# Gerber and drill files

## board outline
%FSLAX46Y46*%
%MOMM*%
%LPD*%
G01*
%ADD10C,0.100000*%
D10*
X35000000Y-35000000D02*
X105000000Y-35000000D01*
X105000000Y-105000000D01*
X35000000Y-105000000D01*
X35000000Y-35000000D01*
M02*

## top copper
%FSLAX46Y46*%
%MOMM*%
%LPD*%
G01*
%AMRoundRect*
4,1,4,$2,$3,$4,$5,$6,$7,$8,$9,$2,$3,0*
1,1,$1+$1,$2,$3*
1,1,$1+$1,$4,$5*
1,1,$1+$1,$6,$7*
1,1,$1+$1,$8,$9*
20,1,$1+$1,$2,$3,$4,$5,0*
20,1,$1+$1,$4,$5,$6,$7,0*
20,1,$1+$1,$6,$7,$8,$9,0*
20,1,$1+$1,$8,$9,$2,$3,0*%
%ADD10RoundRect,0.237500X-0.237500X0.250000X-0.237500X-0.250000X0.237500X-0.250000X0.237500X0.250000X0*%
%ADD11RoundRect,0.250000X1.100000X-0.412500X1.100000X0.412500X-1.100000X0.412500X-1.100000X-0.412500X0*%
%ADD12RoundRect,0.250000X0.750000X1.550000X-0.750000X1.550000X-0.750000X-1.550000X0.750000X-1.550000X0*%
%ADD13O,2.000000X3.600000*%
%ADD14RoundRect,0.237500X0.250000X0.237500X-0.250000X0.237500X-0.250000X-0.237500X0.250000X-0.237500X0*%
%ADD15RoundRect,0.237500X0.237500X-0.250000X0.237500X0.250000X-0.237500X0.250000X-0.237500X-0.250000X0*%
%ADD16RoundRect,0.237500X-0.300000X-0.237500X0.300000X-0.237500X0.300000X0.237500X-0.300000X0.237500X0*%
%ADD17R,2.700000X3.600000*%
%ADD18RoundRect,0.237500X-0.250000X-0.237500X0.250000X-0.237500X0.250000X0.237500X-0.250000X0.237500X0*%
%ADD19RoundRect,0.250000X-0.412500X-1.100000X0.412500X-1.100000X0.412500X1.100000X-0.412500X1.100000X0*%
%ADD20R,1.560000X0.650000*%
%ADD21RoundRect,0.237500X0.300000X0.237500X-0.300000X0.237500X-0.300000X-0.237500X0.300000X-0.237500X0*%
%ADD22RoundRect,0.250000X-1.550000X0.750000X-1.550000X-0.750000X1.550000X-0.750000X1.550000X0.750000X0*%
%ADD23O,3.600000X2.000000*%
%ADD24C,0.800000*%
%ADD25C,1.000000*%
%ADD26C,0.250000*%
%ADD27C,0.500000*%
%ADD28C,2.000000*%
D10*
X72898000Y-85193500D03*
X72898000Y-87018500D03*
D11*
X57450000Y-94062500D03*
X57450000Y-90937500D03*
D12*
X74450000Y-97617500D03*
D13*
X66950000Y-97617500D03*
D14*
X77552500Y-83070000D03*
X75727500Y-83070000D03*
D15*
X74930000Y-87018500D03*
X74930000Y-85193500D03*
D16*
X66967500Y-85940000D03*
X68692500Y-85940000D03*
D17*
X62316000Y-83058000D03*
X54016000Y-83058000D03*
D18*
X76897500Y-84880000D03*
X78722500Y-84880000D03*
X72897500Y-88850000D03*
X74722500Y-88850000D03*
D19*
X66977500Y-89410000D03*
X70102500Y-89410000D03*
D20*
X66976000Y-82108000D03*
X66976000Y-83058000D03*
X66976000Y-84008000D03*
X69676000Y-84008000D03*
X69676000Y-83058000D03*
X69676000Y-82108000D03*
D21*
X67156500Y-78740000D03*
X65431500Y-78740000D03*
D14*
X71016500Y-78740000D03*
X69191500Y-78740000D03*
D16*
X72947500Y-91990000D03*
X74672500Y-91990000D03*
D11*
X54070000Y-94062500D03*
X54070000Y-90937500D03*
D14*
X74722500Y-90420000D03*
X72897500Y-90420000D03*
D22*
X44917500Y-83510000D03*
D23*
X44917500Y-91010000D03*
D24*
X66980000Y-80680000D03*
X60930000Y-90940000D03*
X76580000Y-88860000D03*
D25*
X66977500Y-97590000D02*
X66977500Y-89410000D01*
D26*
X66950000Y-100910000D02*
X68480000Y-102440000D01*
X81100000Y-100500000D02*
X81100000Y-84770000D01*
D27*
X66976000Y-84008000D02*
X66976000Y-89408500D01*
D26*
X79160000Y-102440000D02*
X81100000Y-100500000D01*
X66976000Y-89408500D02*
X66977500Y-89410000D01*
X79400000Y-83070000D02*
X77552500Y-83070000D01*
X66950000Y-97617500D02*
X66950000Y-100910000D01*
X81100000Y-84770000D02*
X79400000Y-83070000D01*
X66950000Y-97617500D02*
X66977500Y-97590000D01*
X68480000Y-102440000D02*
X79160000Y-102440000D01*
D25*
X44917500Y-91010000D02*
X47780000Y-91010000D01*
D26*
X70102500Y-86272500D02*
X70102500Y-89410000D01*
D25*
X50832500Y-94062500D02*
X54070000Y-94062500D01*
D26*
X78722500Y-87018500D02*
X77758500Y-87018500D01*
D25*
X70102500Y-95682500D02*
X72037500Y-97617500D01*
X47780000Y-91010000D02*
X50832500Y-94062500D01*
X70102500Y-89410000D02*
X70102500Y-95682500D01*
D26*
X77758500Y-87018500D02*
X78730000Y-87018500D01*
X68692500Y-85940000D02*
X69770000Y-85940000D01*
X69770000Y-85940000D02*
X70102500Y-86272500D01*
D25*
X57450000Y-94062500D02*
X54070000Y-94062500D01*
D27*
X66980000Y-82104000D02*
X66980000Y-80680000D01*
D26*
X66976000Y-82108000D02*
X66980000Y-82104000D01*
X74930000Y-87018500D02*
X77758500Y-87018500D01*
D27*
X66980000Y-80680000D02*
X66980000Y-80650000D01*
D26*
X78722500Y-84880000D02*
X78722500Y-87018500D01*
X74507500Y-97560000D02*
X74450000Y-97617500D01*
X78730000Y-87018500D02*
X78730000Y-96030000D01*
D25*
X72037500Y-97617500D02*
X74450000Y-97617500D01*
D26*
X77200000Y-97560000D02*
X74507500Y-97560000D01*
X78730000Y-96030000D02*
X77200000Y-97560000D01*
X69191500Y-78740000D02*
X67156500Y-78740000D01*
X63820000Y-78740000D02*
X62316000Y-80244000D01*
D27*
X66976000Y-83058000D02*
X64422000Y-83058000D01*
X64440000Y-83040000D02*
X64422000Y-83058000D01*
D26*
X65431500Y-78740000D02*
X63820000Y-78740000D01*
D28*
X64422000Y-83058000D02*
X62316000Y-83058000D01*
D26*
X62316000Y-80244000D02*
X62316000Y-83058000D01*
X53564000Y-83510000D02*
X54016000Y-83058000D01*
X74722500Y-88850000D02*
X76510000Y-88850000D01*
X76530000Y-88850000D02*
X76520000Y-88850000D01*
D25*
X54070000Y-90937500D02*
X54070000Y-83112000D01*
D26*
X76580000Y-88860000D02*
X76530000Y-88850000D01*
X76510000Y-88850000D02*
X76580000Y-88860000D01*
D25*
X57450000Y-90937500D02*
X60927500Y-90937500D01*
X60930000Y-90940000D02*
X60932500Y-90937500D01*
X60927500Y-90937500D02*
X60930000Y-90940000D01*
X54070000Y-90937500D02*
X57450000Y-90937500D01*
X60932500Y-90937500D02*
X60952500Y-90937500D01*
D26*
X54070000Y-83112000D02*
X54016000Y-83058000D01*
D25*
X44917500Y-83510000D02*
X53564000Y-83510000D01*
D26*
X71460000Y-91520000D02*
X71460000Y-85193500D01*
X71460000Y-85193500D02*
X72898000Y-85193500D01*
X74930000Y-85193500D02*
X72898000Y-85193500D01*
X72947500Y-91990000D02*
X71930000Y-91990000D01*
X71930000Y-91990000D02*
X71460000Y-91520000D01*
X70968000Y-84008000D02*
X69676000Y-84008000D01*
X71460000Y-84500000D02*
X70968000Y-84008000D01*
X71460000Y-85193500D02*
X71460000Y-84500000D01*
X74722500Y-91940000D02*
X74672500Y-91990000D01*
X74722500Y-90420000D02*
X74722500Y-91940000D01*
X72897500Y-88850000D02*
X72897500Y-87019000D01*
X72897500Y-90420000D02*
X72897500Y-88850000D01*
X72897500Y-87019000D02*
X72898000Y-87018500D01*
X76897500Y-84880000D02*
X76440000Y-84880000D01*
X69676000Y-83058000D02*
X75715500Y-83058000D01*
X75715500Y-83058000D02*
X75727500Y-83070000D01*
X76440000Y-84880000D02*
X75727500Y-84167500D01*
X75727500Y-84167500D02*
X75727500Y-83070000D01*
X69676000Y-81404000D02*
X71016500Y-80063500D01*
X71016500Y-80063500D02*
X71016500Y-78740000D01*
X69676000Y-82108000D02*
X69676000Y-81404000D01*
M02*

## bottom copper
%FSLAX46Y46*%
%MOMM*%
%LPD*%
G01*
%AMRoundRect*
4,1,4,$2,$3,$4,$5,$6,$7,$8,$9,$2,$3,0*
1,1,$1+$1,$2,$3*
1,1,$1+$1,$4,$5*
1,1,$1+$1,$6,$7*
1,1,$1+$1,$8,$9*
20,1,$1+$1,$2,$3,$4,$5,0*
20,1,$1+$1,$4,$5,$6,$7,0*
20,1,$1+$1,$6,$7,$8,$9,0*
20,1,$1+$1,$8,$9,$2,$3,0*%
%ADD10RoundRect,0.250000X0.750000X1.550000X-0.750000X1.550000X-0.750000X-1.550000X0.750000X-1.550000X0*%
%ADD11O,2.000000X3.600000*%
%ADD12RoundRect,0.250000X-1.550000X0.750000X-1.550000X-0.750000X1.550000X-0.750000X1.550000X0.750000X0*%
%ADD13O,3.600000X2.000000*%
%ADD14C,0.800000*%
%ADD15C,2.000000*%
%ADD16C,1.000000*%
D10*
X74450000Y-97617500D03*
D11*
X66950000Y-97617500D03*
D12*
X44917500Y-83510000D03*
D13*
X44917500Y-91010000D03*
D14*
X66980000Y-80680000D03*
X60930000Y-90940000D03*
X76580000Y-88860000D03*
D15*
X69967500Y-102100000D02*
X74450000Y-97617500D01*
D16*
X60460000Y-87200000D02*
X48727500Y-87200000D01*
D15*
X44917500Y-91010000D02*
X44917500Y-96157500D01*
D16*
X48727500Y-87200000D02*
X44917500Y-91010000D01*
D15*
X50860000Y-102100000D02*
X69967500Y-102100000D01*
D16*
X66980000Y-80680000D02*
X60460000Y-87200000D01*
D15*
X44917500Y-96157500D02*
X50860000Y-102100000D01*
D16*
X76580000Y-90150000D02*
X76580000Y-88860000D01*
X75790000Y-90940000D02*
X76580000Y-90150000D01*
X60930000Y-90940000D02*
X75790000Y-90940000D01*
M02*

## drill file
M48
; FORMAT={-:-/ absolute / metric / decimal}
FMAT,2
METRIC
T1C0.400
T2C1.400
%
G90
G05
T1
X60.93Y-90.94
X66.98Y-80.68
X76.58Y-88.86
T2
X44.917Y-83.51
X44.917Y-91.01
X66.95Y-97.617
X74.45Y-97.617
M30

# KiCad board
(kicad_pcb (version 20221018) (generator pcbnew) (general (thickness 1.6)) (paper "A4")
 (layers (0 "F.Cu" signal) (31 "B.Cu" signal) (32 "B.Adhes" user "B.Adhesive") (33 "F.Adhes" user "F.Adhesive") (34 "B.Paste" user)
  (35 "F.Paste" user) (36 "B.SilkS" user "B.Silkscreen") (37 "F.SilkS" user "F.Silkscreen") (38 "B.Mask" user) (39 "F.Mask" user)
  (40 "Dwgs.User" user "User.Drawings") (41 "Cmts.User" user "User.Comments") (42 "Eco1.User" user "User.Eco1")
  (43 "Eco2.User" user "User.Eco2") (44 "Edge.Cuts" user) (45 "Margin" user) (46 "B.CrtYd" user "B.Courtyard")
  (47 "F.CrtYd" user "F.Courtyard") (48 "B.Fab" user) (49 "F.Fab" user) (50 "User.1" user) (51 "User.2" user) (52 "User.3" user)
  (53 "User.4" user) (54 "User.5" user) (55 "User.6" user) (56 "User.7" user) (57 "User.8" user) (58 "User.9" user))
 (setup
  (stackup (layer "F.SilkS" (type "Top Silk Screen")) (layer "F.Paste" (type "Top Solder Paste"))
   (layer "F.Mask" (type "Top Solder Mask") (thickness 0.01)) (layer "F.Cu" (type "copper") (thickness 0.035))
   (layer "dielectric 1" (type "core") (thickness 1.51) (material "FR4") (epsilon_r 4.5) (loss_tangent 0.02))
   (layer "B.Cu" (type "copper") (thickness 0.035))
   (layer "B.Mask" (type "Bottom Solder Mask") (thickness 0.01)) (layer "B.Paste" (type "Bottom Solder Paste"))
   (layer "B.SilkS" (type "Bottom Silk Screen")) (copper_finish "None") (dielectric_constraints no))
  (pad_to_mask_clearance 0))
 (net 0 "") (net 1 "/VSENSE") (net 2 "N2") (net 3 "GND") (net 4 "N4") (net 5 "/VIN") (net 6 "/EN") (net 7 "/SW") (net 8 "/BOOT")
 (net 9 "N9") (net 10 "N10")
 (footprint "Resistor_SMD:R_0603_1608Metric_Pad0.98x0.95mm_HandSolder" (layer "F.Cu") (at 72.898 86.106 -90)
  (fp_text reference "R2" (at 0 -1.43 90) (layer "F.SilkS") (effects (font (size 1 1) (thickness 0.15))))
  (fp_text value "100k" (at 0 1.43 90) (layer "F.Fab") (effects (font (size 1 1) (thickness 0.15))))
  (pad "1" smd roundrect (at -0.9125 0 270) (size 0.975 0.95) (layers "F.Cu" "F.Paste" "F.Mask") (roundrect_rratio 0.25) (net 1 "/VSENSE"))
  (pad "2" smd roundrect (at 0.9125 0 270) (size 0.975 0.95) (layers "F.Cu" "F.Paste" "F.Mask") (roundrect_rratio 0.25) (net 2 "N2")))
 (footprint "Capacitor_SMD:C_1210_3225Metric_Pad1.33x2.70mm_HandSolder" (layer "F.Cu") (at 57.45 92.5 90)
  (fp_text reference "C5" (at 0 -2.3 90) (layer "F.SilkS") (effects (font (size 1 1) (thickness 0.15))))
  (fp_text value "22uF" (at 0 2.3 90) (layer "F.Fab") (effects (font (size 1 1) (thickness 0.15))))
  (pad "1" smd roundrect (at -1.5625 0 90) (size 1.325 2.7) (layers "F.Cu" "F.Paste" "F.Mask") (roundrect_rratio 0.188679) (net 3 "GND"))
  (pad "2" smd roundrect (at 1.5625 0 90) (size 1.325 2.7) (layers "F.Cu" "F.Paste" "F.Mask") (roundrect_rratio 0.188679) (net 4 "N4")))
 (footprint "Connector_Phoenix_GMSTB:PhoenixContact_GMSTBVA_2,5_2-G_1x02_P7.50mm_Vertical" (layer "F.Cu") (at 70.76 97.6175 180)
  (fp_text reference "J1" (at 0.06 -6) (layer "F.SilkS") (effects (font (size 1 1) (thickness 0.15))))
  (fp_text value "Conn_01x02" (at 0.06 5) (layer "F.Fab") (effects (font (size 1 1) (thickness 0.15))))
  (pad "1" thru_hole roundrect (at -3.69 0 180) (size 2 3.6) (drill 1.4) (layers "*.Cu" "*.Mask") (roundrect_rratio 0.125) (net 3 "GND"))
  (pad "2" thru_hole oval (at 3.81 0 180) (size 2 3.6) (drill 1.4) (layers "*.Cu" "*.Mask") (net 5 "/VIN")))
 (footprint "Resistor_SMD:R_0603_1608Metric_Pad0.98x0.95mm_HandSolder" (layer "F.Cu") (at 76.64 83.07 180)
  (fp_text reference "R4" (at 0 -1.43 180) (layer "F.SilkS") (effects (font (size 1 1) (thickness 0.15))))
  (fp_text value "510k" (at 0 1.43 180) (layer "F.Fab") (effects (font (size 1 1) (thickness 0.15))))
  (pad "1" smd roundrect (at -0.9125 0 180) (size 0.975 0.95) (layers "F.Cu" "F.Paste" "F.Mask") (roundrect_rratio 0.25) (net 5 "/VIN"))
  (pad "2" smd roundrect (at 0.9125 0 180) (size 0.975 0.95) (layers "F.Cu" "F.Paste" "F.Mask") (roundrect_rratio 0.25) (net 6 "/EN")))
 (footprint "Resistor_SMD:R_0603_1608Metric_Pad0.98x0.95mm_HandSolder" (layer "F.Cu") (at 74.93 86.106 90)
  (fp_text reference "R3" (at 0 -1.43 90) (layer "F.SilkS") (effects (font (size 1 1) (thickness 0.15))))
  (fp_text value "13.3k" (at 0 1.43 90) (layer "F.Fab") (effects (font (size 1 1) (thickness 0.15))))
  (pad "1" smd roundrect (at -0.9125 0 90) (size 0.975 0.95) (layers "F.Cu" "F.Paste" "F.Mask") (roundrect_rratio 0.25) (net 3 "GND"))
  (pad "2" smd roundrect (at 0.9125 0 90) (size 0.975 0.95) (layers "F.Cu" "F.Paste" "F.Mask") (roundrect_rratio 0.25) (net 1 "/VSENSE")))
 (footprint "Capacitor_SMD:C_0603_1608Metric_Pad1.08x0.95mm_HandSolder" (layer "F.Cu") (at 67.83 85.94)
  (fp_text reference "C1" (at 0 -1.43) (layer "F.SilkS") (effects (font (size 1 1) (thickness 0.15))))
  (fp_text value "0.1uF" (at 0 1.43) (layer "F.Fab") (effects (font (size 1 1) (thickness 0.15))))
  (pad "1" smd roundrect (at -0.8625 0) (size 1.075 0.95) (layers "F.Cu" "F.Paste" "F.Mask") (roundrect_rratio 0.25) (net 5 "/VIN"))
  (pad "2" smd roundrect (at 0.8625 0) (size 1.075 0.95) (layers "F.Cu" "F.Paste" "F.Mask") (roundrect_rratio 0.25) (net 3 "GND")))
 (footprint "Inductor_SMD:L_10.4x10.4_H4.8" (layer "F.Cu") (at 58.166 83.058 180)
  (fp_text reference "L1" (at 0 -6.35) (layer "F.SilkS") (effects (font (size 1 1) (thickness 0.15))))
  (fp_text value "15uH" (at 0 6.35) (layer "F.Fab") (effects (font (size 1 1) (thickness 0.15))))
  (pad "1" smd rect (at -4.15 0 180) (size 2.7 3.6) (layers "F.Cu" "F.Paste" "F.Mask") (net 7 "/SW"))
  (pad "2" smd rect (at 4.15 0 180) (size 2.7 3.6) (layers "F.Cu" "F.Paste" "F.Mask") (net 4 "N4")))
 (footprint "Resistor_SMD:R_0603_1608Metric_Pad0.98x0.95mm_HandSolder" (layer "F.Cu") (at 77.81 84.88)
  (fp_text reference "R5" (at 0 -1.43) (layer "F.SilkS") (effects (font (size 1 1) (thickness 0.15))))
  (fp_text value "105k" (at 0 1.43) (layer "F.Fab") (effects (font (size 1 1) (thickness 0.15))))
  (pad "1" smd roundrect (at -0.9125 0) (size 0.975 0.95) (layers "F.Cu" "F.Paste" "F.Mask") (roundrect_rratio 0.25) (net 6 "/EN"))
  (pad "2" smd roundrect (at 0.9125 0) (size 0.975 0.95) (layers "F.Cu" "F.Paste" "F.Mask") (roundrect_rratio 0.25) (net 3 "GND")))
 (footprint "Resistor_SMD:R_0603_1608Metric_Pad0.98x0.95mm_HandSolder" (layer "F.Cu") (at 73.81 88.85)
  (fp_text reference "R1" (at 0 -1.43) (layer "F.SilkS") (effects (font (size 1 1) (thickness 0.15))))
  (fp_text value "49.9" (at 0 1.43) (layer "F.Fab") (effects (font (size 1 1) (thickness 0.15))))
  (pad "1" smd roundrect (at -0.9125 0) (size 0.975 0.95) (layers "F.Cu" "F.Paste" "F.Mask") (roundrect_rratio 0.25) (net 2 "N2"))
  (pad "2" smd roundrect (at 0.9125 0) (size 0.975 0.95) (layers "F.Cu" "F.Paste" "F.Mask") (roundrect_rratio 0.25) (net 4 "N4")))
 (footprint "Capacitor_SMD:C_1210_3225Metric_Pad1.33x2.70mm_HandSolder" (layer "F.Cu") (at 68.54 89.41)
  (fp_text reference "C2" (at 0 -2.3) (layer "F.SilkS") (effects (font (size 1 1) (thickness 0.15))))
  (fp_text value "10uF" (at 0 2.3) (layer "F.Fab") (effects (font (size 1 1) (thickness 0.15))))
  (pad "1" smd roundrect (at -1.5625 0) (size 1.325 2.7) (layers "F.Cu" "F.Paste" "F.Mask") (roundrect_rratio 0.188679) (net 5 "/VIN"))
  (pad "2" smd roundrect (at 1.5625 0) (size 1.325 2.7) (layers "F.Cu" "F.Paste" "F.Mask") (roundrect_rratio 0.188679) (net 3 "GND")))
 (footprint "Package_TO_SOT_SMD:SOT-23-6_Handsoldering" (layer "F.Cu") (at 68.326 83.058)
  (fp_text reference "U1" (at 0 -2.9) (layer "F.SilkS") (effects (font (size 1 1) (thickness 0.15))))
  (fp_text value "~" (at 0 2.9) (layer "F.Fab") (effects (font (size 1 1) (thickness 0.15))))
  (pad "1" smd rect (at -1.35 -0.95) (size 1.56 0.65) (layers "F.Cu" "F.Paste" "F.Mask") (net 3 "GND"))
  (pad "2" smd rect (at -1.35 0) (size 1.56 0.65) (layers "F.Cu" "F.Paste" "F.Mask") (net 7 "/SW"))
  (pad "3" smd rect (at -1.35 0.95) (size 1.56 0.65) (layers "F.Cu" "F.Paste" "F.Mask") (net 5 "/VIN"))
  (pad "4" smd rect (at 1.35 0.95) (size 1.56 0.65) (layers "F.Cu" "F.Paste" "F.Mask") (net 1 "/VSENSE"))
  (pad "5" smd rect (at 1.35 0) (size 1.56 0.65) (layers "F.Cu" "F.Paste" "F.Mask") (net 6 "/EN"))
  (pad "6" smd rect (at 1.35 -0.95) (size 1.56 0.65) (layers "F.Cu" "F.Paste" "F.Mask") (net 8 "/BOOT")))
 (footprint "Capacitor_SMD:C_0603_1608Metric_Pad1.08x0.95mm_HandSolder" (layer "F.Cu") (at 66.294 78.74 180)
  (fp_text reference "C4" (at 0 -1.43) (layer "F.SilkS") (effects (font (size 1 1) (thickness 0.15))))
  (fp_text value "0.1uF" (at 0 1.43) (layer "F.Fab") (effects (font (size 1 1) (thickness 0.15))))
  (pad "1" smd roundrect (at -0.8625 0 180) (size 1.075 0.95) (layers "F.Cu" "F.Paste" "F.Mask") (roundrect_rratio 0.25) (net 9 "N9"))
  (pad "2" smd roundrect (at 0.8625 0 180) (size 1.075 0.95) (layers "F.Cu" "F.Paste" "F.Mask") (roundrect_rratio 0.25) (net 7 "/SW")))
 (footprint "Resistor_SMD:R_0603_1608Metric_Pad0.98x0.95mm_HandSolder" (layer "F.Cu") (at 70.104 78.74 180)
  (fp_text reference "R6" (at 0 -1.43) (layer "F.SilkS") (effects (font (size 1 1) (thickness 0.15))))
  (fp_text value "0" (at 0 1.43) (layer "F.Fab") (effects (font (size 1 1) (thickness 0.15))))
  (pad "1" smd roundrect (at -0.9125 0 180) (size 0.975 0.95) (layers "F.Cu" "F.Paste" "F.Mask") (roundrect_rratio 0.25) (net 8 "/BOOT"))
  (pad "2" smd roundrect (at 0.9125 0 180) (size 0.975 0.95) (layers "F.Cu" "F.Paste" "F.Mask") (roundrect_rratio 0.25) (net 9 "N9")))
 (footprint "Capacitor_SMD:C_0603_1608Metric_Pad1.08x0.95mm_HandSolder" (layer "F.Cu") (at 73.81 91.99)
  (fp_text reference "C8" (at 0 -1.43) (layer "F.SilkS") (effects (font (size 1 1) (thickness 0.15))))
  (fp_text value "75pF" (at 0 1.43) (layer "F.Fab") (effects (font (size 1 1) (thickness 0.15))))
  (pad "1" smd roundrect (at -0.8625 0) (size 1.075 0.95) (layers "F.Cu" "F.Paste" "F.Mask") (roundrect_rratio 0.25) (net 1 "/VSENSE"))
  (pad "2" smd roundrect (at 0.8625 0) (size 1.075 0.95) (layers "F.Cu" "F.Paste" "F.Mask") (roundrect_rratio 0.25) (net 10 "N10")))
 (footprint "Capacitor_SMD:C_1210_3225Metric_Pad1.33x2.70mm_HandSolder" (layer "F.Cu") (at 54.07 92.5 90)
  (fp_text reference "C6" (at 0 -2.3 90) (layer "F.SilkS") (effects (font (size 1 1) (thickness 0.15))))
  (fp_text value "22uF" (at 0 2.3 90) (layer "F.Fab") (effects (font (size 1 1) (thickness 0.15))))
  (pad "1" smd roundrect (at -1.5625 0 90) (size 1.325 2.7) (layers "F.Cu" "F.Paste" "F.Mask") (roundrect_rratio 0.188679) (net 3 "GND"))
  (pad "2" smd roundrect (at 1.5625 0 90) (size 1.325 2.7) (layers "F.Cu" "F.Paste" "F.Mask") (roundrect_rratio 0.188679) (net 4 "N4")))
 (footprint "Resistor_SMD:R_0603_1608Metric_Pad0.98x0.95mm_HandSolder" (layer "F.Cu") (at 73.81 90.42 180)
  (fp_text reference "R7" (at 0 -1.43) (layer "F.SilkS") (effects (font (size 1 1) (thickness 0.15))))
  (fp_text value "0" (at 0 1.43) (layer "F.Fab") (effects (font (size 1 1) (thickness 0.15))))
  (pad "1" smd roundrect (at -0.9125 0 180) (size 0.975 0.95) (layers "F.Cu" "F.Paste" "F.Mask") (roundrect_rratio 0.25) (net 10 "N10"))
  (pad "2" smd roundrect (at 0.9125 0 180) (size 0.975 0.95) (layers "F.Cu" "F.Paste" "F.Mask") (roundrect_rratio 0.25) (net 2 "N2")))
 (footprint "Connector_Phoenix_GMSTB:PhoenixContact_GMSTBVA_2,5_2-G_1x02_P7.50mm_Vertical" (layer "F.Cu") (at 44.9175 87.2 -90)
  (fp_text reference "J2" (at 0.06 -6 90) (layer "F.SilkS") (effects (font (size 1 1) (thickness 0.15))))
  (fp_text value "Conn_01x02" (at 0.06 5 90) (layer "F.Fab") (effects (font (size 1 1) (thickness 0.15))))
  (pad "1" thru_hole roundrect (at -3.69 0 270) (size 2 3.6) (drill 1.4) (layers "*.Cu" "*.Mask") (roundrect_rratio 0.125) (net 4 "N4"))
  (pad "2" thru_hole oval (at 3.81 0 270) (size 2 3.6) (drill 1.4) (layers "*.Cu" "*.Mask") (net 3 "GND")))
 (gr_rect (start 35 35) (end 105 105) (stroke (width 0.1) (type default)) (fill none) (layer "Edge.Cuts"))
 (segment (start 66.9775 97.59) (end 66.9775 89.41) (width 1) (layer "F.Cu") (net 5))
 (segment (start 66.95 100.91) (end 68.48 102.44) (width 0.25) (layer "F.Cu") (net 5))
 (segment (start 81.1 100.5) (end 81.1 84.77) (width 0.25) (layer "F.Cu") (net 5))
 (segment (start 66.976 84.008) (end 66.976 89.4085) (width 0.5) (layer "F.Cu") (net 5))
 (segment (start 79.16 102.44) (end 81.1 100.5) (width 0.25) (layer "F.Cu") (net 5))
 (segment (start 66.976 89.4085) (end 66.9775 89.41) (width 0.25) (layer "F.Cu") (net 5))
 (segment (start 79.4 83.07) (end 77.5525 83.07) (width 0.25) (layer "F.Cu") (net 5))
 (segment (start 66.95 97.6175) (end 66.95 100.91) (width 0.25) (layer "F.Cu") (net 5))
 (segment (start 81.1 84.77) (end 79.4 83.07) (width 0.25) (layer "F.Cu") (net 5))
 (segment (start 66.95 97.6175) (end 66.9775 97.59) (width 0.25) (layer "F.Cu") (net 5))
 (segment (start 68.48 102.44) (end 79.16 102.44) (width 0.25) (layer "F.Cu") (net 5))
 (segment (start 44.9175 91.01) (end 47.78 91.01) (width 1) (layer "F.Cu") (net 3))
 (segment (start 70.1025 86.2725) (end 70.1025 89.41) (width 0.25) (layer "F.Cu") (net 3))
 (segment (start 50.8325 94.0625) (end 54.07 94.0625) (width 1) (layer "F.Cu") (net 3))
 (segment (start 78.7225 87.0185) (end 77.7585 87.0185) (width 0.25) (layer "F.Cu") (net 3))
 (segment (start 70.1025 95.6825) (end 72.0375 97.6175) (width 1) (layer "F.Cu") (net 3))
 (segment (start 47.78 91.01) (end 50.8325 94.0625) (width 1) (layer "F.Cu") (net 3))
 (segment (start 70.1025 89.41) (end 70.1025 95.6825) (width 1) (layer "F.Cu") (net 3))
 (segment (start 77.7585 87.0185) (end 78.73 87.0185) (width 0.25) (layer "F.Cu") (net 3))
 (segment (start 68.6925 85.94) (end 69.77 85.94) (width 0.25) (layer "F.Cu") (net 3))
 (segment (start 69.77 85.94) (end 70.1025 86.2725) (width 0.25) (layer "F.Cu") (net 3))
 (segment (start 57.45 94.0625) (end 54.07 94.0625) (width 1) (layer "F.Cu") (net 3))
 (segment (start 66.98 82.104) (end 66.98 80.68) (width 0.5) (layer "F.Cu") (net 3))
 (segment (start 66.976 82.108) (end 66.98 82.104) (width 0.25) (layer "F.Cu") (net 3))
 (segment (start 74.93 87.0185) (end 77.7585 87.0185) (width 0.25) (layer "F.Cu") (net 3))
 (segment (start 66.98 80.68) (end 66.98 80.65) (width 0.5) (layer "F.Cu") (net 3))
 (segment (start 78.7225 84.88) (end 78.7225 87.0185) (width 0.25) (layer "F.Cu") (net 3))
 (segment (start 74.5075 97.56) (end 74.45 97.6175) (width 0.25) (layer "F.Cu") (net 3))
 (segment (start 78.73 87.0185) (end 78.73 96.03) (width 0.25) (layer "F.Cu") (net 3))
 (segment (start 72.0375 97.6175) (end 74.45 97.6175) (width 1) (layer "F.Cu") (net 3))
 (segment (start 77.2 97.56) (end 74.5075 97.56) (width 0.25) (layer "F.Cu") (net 3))
 (segment (start 78.73 96.03) (end 77.2 97.56) (width 0.25) (layer "F.Cu") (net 3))
 (via (at 66.98 80.68) (size 0.8) (drill 0.4) (layers "F.Cu" "B.Cu") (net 3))
 (segment (start 69.9675 102.1) (end 74.45 97.6175) (width 2) (layer "B.Cu") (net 3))
 (segment (start 60.46 87.2) (end 48.7275 87.2) (width 1) (layer "B.Cu") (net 3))
 (segment (start 44.9175 91.01) (end 44.9175 96.1575) (width 2) (layer "B.Cu") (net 3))
 (segment (start 48.7275 87.2) (end 44.9175 91.01) (width 1) (layer "B.Cu") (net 3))
 (segment (start 50.86 102.1) (end 69.9675 102.1) (width 2) (layer "B.Cu") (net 3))
 (segment (start 66.98 80.68) (end 60.46 87.2) (width 1) (layer "B.Cu") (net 3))
 (segment (start 44.9175 96.1575) (end 50.86 102.1) (width 2) (layer "B.Cu") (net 3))
 (segment (start 69.1915 78.74) (end 67.1565 78.74) (width 0.25) (layer "F.Cu") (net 9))
 (segment (start 63.82 78.74) (end 62.316 80.244) (width 0.25) (layer "F.Cu") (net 7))
 (segment (start 66.976 83.058) (end 64.422 83.058) (width 0.5) (layer "F.Cu") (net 7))
 (segment (start 64.44 83.04) (end 64.422 83.058) (width 0.5) (layer "F.Cu") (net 7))
 (segment (start 65.4315 78.74) (end 63.82 78.74) (width 0.25) (layer "F.Cu") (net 7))
 (segment (start 64.422 83.058) (end 62.316 83.058) (width 2) (layer "F.Cu") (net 7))
 (segment (start 62.316 80.244) (end 62.316 83.058) (width 0.25) (layer "F.Cu") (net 7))
 (segment (start 53.564 83.51) (end 54.016 83.058) (width 0.25) (layer "F.Cu") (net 4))
 (segment (start 74.7225 88.85) (end 76.51 88.85) (width 0.25) (layer "F.Cu") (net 4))
 (segment (start 76.53 88.85) (end 76.52 88.85) (width 0.25) (layer "F.Cu") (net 4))
 (segment (start 54.07 90.9375) (end 54.07 83.112) (width 1) (layer "F.Cu") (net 4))
 (segment (start 76.58 88.86) (end 76.53 88.85) (width 0.25) (layer "F.Cu") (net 4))
 (segment (start 76.51 88.85) (end 76.58 88.86) (width 0.25) (layer "F.Cu") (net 4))
 (segment (start 57.45 90.9375) (end 60.9275 90.9375) (width 1) (layer "F.Cu") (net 4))
 (segment (start 60.93 90.94) (end 60.9325 90.9375) (width 1) (layer "F.Cu") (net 4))
 (segment (start 60.9275 90.9375) (end 60.93 90.94) (width 1) (layer "F.Cu") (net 4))
 (segment (start 54.07 90.9375) (end 57.45 90.9375) (width 1) (layer "F.Cu") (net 4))
 (segment (start 60.9325 90.9375) (end 60.9525 90.9375) (width 1) (layer "F.Cu") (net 4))
 (segment (start 54.07 83.112) (end 54.016 83.058) (width 0.25) (layer "F.Cu") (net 4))
 (segment (start 44.9175 83.51) (end 53.564 83.51) (width 1) (layer "F.Cu") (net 4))
 (via (at 60.93 90.94) (size 0.8) (drill 0.4) (layers "F.Cu" "B.Cu") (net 4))
 (via (at 76.58 88.86) (size 0.8) (drill 0.4) (layers "F.Cu" "B.Cu") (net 4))
 (segment (start 76.58 90.15) (end 76.58 88.86) (width 1) (layer "B.Cu") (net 4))
 (segment (start 75.79 90.94) (end 76.58 90.15) (width 1) (layer "B.Cu") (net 4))
 (segment (start 60.93 90.94) (end 75.79 90.94) (width 1) (layer "B.Cu") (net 4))
 (segment (start 71.46 91.52) (end 71.46 85.1935) (width 0.25) (layer "F.Cu") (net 1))
 (segment (start 71.46 85.1935) (end 72.898 85.1935) (width 0.25) (layer "F.Cu") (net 1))
 (segment (start 74.93 85.1935) (end 72.898 85.1935) (width 0.25) (layer "F.Cu") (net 1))
 (segment (start 72.9475 91.99) (end 71.93 91.99) (width 0.25) (layer "F.Cu") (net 1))
 (segment (start 71.93 91.99) (end 71.46 91.52) (width 0.25) (layer "F.Cu") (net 1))
 (segment (start 70.968 84.008) (end 69.676 84.008) (width 0.25) (layer "F.Cu") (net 1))
 (segment (start 71.46 84.5) (end 70.968 84.008) (width 0.25) (layer "F.Cu") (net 1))
 (segment (start 71.46 85.1935) (end 71.46 84.5) (width 0.25) (layer "F.Cu") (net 1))
 (segment (start 74.7225 91.94) (end 74.6725 91.99) (width 0.25) (layer "F.Cu") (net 10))
 (segment (start 74.7225 90.42) (end 74.7225 91.94) (width 0.25) (layer "F.Cu") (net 10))
 (segment (start 72.8975 88.85) (end 72.8975 87.019) (width 0.25) (layer "F.Cu") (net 2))
 (segment (start 72.8975 90.42) (end 72.8975 88.85) (width 0.25) (layer "F.Cu") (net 2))
 (segment (start 72.8975 87.019) (end 72.898 87.0185) (width 0.25) (layer "F.Cu") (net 2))
 (segment (start 76.8975 84.88) (end 76.44 84.88) (width 0.25) (layer "F.Cu") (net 6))
 (segment (start 69.676 83.058) (end 75.7155 83.058) (width 0.25) (layer "F.Cu") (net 6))
 (segment (start 75.7155 83.058) (end 75.7275 83.07) (width 0.25) (layer "F.Cu") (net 6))
 (segment (start 76.44 84.88) (end 75.7275 84.1675) (width 0.25) (layer "F.Cu") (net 6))
 (segment (start 75.7275 84.1675) (end 75.7275 83.07) (width 0.25) (layer "F.Cu") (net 6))
 (segment (start 69.676 81.404) (end 71.0165 80.0635) (width 0.25) (layer "F.Cu") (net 8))
 (segment (start 71.0165 80.0635) (end 71.0165 78.74) (width 0.25) (layer "F.Cu") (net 8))
 (segment (start 69.676 82.108) (end 69.676 81.404) (width 0.25) (layer "F.Cu") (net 8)))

